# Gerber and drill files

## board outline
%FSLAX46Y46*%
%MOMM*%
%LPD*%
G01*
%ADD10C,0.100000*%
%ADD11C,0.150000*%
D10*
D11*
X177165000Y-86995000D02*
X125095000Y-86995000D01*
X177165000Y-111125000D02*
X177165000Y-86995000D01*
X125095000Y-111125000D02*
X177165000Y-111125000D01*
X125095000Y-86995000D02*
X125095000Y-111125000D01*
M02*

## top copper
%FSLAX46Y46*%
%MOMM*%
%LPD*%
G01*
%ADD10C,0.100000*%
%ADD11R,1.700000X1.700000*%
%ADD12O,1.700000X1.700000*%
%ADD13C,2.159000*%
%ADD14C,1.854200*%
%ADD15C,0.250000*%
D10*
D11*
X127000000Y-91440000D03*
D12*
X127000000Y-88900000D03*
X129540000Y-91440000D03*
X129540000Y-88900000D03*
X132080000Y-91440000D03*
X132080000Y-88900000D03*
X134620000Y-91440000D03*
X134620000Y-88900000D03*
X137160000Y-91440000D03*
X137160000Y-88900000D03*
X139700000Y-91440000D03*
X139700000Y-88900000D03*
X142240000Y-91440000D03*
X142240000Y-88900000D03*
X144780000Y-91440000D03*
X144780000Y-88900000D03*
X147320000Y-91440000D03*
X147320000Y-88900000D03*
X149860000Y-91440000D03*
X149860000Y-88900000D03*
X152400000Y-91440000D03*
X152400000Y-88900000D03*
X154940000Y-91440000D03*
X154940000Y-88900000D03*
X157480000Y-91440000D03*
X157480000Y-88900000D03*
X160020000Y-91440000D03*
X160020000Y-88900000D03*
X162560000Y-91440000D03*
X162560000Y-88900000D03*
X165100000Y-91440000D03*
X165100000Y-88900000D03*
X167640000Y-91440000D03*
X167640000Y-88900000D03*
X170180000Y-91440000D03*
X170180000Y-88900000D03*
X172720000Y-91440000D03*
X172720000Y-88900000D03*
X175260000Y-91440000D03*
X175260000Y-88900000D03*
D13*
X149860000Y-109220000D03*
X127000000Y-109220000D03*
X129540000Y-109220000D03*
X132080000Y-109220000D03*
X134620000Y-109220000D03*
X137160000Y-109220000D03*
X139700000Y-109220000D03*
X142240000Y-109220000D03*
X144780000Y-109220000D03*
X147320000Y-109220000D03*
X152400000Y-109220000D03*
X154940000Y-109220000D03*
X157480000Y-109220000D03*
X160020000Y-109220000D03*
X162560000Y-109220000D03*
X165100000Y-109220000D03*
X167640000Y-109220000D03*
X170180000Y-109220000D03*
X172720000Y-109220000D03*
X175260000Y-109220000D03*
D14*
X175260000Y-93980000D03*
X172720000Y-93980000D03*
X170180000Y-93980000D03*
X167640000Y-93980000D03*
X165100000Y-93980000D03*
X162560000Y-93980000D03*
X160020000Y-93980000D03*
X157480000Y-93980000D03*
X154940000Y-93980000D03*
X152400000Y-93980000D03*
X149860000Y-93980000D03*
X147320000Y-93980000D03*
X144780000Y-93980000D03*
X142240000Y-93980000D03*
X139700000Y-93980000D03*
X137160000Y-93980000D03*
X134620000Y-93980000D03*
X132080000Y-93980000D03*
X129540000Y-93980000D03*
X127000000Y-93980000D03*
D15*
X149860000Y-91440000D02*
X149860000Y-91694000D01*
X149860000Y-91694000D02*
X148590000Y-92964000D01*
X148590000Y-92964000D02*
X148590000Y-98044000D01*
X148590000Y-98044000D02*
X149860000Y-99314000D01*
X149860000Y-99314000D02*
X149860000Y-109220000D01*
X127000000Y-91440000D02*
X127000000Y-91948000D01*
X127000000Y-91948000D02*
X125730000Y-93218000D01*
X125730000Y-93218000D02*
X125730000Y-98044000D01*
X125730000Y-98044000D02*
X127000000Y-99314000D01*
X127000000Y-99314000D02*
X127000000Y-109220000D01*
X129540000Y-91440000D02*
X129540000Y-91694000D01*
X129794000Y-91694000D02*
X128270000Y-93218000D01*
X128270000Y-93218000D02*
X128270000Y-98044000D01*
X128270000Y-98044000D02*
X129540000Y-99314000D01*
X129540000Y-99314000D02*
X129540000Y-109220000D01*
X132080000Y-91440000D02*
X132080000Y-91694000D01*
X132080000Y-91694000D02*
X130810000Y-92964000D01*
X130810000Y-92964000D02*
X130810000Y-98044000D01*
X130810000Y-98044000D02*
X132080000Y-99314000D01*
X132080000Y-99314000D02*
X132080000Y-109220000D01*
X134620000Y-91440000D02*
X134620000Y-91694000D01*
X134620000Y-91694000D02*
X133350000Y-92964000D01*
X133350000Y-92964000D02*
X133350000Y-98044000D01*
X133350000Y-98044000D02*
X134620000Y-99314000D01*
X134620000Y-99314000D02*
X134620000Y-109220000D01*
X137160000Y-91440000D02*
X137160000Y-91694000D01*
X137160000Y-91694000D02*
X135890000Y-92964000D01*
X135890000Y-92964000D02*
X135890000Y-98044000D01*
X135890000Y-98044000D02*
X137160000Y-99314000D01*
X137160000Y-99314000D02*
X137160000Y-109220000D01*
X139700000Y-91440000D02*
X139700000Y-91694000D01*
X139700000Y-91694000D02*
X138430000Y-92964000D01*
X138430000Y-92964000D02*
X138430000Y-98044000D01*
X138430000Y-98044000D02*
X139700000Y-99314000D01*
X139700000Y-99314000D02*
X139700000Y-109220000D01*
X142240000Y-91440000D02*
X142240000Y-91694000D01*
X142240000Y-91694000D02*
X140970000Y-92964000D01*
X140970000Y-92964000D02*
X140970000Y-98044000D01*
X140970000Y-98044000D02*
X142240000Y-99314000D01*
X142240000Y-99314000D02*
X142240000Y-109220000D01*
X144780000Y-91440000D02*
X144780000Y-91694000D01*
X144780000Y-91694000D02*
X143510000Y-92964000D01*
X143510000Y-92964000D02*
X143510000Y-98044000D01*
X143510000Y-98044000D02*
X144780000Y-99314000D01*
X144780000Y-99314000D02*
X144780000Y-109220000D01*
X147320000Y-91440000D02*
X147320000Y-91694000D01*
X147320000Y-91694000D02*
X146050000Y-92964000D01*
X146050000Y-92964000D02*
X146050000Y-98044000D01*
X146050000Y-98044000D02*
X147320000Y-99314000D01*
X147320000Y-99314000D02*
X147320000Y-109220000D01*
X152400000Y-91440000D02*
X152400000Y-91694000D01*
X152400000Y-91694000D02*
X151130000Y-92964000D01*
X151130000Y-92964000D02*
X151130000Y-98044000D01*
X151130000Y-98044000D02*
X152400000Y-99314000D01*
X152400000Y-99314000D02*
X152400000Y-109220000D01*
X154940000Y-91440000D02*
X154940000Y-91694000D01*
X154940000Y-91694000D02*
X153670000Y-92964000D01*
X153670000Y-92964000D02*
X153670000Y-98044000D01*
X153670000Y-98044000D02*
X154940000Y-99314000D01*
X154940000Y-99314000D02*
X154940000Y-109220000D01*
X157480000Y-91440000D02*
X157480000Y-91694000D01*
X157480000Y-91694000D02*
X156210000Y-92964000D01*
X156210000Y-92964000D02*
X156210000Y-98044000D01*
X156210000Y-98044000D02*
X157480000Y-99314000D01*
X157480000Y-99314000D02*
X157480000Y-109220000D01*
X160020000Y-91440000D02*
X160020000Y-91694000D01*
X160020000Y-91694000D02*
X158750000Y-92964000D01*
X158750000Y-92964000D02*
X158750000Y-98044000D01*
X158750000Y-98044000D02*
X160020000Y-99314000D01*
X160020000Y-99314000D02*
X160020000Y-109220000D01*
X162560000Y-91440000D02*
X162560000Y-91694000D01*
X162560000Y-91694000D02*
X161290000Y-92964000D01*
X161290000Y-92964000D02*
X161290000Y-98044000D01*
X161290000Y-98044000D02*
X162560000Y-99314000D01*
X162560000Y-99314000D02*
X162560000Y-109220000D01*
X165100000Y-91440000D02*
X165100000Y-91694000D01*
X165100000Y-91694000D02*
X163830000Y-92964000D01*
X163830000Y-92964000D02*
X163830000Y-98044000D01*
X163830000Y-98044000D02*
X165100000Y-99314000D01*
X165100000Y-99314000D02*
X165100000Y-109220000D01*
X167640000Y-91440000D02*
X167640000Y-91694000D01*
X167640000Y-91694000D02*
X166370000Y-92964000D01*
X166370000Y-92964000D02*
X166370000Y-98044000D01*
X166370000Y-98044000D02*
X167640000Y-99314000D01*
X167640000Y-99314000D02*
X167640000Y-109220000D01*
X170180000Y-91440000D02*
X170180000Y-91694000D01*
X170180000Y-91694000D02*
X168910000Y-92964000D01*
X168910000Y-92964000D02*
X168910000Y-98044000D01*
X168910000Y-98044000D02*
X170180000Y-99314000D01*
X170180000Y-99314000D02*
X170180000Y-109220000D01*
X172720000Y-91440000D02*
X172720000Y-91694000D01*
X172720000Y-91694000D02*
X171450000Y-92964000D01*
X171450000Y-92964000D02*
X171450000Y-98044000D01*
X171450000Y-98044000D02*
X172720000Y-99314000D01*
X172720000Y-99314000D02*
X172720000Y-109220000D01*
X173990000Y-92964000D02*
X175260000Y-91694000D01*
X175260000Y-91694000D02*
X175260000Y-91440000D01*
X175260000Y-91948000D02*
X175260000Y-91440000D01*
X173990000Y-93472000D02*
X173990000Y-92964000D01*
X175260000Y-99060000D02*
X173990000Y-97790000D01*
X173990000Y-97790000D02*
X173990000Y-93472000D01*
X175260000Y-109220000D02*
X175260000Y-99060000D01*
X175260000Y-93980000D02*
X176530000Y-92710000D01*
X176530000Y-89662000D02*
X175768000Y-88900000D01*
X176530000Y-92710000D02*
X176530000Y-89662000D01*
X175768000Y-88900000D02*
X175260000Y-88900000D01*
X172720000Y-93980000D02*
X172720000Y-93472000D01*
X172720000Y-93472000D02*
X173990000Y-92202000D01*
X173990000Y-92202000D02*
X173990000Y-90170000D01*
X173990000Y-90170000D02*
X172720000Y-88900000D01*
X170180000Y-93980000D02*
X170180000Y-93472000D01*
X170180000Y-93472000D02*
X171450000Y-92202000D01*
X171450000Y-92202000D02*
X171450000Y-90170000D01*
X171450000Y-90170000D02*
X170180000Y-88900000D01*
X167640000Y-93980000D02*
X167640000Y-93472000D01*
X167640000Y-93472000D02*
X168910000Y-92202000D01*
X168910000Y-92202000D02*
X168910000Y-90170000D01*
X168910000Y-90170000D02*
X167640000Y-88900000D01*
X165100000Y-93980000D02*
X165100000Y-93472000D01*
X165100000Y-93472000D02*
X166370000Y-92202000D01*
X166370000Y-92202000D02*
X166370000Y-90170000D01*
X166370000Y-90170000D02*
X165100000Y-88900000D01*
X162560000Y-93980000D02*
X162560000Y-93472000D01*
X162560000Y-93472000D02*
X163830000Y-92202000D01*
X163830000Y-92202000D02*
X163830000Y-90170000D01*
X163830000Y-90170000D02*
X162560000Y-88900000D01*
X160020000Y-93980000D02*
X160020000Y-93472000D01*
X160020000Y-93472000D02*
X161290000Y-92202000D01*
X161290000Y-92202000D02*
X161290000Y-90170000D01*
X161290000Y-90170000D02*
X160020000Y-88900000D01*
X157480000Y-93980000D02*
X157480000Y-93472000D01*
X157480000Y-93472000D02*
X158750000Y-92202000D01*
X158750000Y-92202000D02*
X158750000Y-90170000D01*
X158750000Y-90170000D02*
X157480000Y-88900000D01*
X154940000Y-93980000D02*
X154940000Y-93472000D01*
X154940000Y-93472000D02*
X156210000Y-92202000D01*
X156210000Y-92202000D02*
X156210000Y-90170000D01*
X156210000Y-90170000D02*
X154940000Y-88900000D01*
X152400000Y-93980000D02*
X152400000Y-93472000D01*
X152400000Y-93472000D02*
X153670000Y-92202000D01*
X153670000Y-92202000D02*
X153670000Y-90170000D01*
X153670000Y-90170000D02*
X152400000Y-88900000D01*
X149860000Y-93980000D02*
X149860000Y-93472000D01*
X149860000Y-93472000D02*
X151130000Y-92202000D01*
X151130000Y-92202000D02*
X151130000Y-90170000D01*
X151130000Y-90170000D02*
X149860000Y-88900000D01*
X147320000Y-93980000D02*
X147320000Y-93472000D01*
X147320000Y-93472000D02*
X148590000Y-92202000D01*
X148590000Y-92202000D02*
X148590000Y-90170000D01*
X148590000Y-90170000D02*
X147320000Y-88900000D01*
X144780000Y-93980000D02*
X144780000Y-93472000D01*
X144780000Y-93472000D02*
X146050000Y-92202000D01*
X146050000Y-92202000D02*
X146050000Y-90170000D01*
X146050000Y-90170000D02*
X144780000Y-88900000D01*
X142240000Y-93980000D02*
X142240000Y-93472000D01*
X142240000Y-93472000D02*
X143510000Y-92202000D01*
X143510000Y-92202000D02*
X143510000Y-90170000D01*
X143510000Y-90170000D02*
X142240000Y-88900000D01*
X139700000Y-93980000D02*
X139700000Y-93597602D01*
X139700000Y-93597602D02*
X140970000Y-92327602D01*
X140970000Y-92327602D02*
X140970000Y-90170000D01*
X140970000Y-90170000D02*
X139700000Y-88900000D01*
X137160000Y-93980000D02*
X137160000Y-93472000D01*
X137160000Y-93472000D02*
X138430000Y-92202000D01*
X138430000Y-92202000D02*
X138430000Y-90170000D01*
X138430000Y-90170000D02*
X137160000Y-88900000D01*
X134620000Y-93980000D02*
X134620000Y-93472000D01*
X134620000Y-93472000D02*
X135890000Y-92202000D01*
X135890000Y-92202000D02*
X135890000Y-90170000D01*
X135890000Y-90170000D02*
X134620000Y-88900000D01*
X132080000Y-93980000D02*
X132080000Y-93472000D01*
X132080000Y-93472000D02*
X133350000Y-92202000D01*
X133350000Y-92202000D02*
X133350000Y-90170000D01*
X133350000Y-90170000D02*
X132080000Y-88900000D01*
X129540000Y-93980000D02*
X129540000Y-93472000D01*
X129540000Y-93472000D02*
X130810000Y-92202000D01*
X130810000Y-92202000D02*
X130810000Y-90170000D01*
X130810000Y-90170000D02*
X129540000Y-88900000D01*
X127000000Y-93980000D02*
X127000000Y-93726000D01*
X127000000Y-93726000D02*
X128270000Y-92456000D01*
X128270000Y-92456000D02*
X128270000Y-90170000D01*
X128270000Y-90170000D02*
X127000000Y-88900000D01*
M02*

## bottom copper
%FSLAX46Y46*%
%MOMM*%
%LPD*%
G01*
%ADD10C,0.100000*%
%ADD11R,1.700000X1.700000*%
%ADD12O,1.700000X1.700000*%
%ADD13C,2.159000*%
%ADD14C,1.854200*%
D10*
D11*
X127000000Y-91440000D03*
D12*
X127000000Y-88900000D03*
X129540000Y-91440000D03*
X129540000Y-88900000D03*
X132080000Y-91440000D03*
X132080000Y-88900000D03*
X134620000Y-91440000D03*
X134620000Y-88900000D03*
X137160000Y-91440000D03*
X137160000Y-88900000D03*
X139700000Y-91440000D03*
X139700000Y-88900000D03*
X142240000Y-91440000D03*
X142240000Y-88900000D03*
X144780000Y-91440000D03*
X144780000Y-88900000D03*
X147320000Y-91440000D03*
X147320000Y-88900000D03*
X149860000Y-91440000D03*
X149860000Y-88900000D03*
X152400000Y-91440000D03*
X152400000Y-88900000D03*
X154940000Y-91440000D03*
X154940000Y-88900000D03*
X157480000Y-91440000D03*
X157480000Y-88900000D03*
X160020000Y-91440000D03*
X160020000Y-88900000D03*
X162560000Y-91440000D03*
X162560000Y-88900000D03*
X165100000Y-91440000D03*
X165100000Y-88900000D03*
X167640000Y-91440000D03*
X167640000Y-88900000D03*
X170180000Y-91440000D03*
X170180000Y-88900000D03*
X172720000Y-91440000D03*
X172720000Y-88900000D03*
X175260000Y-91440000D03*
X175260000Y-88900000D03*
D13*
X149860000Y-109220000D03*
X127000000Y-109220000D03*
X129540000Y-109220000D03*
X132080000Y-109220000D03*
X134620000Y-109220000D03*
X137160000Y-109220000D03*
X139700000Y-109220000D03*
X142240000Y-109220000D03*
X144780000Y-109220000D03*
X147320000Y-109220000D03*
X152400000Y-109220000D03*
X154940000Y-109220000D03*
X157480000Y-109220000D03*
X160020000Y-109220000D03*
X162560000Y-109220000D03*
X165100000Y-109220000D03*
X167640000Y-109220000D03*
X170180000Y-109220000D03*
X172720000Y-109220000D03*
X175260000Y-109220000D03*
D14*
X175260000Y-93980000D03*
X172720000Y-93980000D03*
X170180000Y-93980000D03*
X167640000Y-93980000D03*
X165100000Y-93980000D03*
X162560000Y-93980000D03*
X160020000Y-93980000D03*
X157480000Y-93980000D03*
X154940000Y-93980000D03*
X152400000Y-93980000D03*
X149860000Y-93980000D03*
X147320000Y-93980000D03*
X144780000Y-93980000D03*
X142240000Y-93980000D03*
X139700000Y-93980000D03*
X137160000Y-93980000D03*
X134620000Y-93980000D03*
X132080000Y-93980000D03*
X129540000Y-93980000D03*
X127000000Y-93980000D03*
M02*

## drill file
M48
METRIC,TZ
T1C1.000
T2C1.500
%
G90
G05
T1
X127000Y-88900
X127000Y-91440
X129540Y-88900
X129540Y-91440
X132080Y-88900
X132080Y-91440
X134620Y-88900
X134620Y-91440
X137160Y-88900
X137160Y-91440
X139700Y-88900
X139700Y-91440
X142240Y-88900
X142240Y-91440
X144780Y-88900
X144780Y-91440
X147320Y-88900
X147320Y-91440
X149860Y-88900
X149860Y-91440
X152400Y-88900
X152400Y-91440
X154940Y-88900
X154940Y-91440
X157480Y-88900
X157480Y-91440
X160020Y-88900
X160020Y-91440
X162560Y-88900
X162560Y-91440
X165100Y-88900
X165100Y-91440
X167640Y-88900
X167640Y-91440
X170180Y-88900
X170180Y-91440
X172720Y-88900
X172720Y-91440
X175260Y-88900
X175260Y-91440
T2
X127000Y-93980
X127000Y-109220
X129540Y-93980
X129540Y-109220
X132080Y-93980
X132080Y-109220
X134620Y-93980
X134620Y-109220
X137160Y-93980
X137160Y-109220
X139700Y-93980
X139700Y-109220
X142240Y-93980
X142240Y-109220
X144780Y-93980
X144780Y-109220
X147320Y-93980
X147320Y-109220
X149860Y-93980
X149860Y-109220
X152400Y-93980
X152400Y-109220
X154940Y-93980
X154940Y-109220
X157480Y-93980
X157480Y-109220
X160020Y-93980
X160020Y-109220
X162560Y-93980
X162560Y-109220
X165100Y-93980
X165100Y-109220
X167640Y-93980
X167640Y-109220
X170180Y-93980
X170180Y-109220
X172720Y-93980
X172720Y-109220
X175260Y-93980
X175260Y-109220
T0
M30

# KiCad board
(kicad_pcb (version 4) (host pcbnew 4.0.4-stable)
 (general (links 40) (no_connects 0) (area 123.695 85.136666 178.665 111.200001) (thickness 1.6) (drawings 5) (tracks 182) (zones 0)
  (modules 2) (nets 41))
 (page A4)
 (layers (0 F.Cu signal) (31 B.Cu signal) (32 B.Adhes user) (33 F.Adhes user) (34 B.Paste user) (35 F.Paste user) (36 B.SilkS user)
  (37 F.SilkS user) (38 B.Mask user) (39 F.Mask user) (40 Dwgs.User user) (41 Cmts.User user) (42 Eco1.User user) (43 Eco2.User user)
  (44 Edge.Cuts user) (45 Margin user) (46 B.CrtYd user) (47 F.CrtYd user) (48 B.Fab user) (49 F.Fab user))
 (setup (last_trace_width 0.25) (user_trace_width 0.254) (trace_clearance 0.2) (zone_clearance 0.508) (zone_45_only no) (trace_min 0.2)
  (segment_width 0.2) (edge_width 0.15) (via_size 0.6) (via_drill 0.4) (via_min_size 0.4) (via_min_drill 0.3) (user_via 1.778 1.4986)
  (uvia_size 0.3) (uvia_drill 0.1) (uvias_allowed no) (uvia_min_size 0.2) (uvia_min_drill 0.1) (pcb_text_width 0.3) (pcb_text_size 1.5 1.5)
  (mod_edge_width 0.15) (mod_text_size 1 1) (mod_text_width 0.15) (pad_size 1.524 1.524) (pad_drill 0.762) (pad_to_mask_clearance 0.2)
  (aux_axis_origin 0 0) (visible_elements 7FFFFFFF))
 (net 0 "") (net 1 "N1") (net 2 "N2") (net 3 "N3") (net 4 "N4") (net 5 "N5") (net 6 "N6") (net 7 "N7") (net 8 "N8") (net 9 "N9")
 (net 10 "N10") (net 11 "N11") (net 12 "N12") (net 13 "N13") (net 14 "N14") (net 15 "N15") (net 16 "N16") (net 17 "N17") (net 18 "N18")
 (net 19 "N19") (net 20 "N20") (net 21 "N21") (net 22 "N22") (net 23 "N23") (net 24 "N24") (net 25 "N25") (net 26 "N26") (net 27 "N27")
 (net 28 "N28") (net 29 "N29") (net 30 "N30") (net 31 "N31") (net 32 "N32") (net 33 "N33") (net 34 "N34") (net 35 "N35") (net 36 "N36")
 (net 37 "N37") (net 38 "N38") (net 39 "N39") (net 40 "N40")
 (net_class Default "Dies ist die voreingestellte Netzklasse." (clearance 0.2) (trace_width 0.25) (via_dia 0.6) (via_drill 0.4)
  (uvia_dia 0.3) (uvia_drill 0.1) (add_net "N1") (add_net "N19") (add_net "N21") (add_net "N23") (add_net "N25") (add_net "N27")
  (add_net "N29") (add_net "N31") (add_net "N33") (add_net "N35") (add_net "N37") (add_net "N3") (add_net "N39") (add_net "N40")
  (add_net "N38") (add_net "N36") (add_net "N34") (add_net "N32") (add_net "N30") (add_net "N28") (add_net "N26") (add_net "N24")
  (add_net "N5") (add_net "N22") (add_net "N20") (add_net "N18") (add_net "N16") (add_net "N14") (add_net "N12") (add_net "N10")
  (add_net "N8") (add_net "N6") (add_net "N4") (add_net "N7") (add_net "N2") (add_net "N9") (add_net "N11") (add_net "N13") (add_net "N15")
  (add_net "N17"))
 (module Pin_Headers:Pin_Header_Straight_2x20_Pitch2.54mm (layer F.Cu) (at 127 91.44 90)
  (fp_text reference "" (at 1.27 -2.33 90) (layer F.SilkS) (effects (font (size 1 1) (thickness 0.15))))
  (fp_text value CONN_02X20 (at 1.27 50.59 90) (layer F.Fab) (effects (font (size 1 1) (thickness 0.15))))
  (pad 1 thru_hole rect (at 0 0 90) (size 1.7 1.7) (drill 1) (layers *.Cu *.Mask) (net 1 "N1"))
  (pad 2 thru_hole oval (at 2.54 0 90) (size 1.7 1.7) (drill 1) (layers *.Cu *.Mask) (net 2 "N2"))
  (pad 3 thru_hole oval (at 0 2.54 90) (size 1.7 1.7) (drill 1) (layers *.Cu *.Mask) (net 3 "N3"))
  (pad 4 thru_hole oval (at 2.54 2.54 90) (size 1.7 1.7) (drill 1) (layers *.Cu *.Mask) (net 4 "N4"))
  (pad 5 thru_hole oval (at 0 5.08 90) (size 1.7 1.7) (drill 1) (layers *.Cu *.Mask) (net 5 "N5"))
  (pad 6 thru_hole oval (at 2.54 5.08 90) (size 1.7 1.7) (drill 1) (layers *.Cu *.Mask) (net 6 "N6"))
  (pad 7 thru_hole oval (at 0 7.62 90) (size 1.7 1.7) (drill 1) (layers *.Cu *.Mask) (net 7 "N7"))
  (pad 8 thru_hole oval (at 2.54 7.62 90) (size 1.7 1.7) (drill 1) (layers *.Cu *.Mask) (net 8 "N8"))
  (pad 9 thru_hole oval (at 0 10.16 90) (size 1.7 1.7) (drill 1) (layers *.Cu *.Mask) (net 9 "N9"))
  (pad 10 thru_hole oval (at 2.54 10.16 90) (size 1.7 1.7) (drill 1) (layers *.Cu *.Mask) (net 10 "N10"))
  (pad 11 thru_hole oval (at 0 12.7 90) (size 1.7 1.7) (drill 1) (layers *.Cu *.Mask) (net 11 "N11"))
  (pad 12 thru_hole oval (at 2.54 12.7 90) (size 1.7 1.7) (drill 1) (layers *.Cu *.Mask) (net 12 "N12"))
  (pad 13 thru_hole oval (at 0 15.24 90) (size 1.7 1.7) (drill 1) (layers *.Cu *.Mask) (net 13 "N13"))
  (pad 14 thru_hole oval (at 2.54 15.24 90) (size 1.7 1.7) (drill 1) (layers *.Cu *.Mask) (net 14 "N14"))
  (pad 15 thru_hole oval (at 0 17.78 90) (size 1.7 1.7) (drill 1) (layers *.Cu *.Mask) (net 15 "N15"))
  (pad 16 thru_hole oval (at 2.54 17.78 90) (size 1.7 1.7) (drill 1) (layers *.Cu *.Mask) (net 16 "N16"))
  (pad 17 thru_hole oval (at 0 20.32 90) (size 1.7 1.7) (drill 1) (layers *.Cu *.Mask) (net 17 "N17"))
  (pad 18 thru_hole oval (at 2.54 20.32 90) (size 1.7 1.7) (drill 1) (layers *.Cu *.Mask) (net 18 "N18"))
  (pad 19 thru_hole oval (at 0 22.86 90) (size 1.7 1.7) (drill 1) (layers *.Cu *.Mask) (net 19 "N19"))
  (pad 20 thru_hole oval (at 2.54 22.86 90) (size 1.7 1.7) (drill 1) (layers *.Cu *.Mask) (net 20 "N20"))
  (pad 21 thru_hole oval (at 0 25.4 90) (size 1.7 1.7) (drill 1) (layers *.Cu *.Mask) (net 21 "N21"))
  (pad 22 thru_hole oval (at 2.54 25.4 90) (size 1.7 1.7) (drill 1) (layers *.Cu *.Mask) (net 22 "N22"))
  (pad 23 thru_hole oval (at 0 27.94 90) (size 1.7 1.7) (drill 1) (layers *.Cu *.Mask) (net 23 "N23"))
  (pad 24 thru_hole oval (at 2.54 27.94 90) (size 1.7 1.7) (drill 1) (layers *.Cu *.Mask) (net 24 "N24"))
  (pad 25 thru_hole oval (at 0 30.48 90) (size 1.7 1.7) (drill 1) (layers *.Cu *.Mask) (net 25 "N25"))
  (pad 26 thru_hole oval (at 2.54 30.48 90) (size 1.7 1.7) (drill 1) (layers *.Cu *.Mask) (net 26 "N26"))
  (pad 27 thru_hole oval (at 0 33.02 90) (size 1.7 1.7) (drill 1) (layers *.Cu *.Mask) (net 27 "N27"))
  (pad 28 thru_hole oval (at 2.54 33.02 90) (size 1.7 1.7) (drill 1) (layers *.Cu *.Mask) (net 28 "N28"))
  (pad 29 thru_hole oval (at 0 35.56 90) (size 1.7 1.7) (drill 1) (layers *.Cu *.Mask) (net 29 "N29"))
  (pad 30 thru_hole oval (at 2.54 35.56 90) (size 1.7 1.7) (drill 1) (layers *.Cu *.Mask) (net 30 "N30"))
  (pad 31 thru_hole oval (at 0 38.1 90) (size 1.7 1.7) (drill 1) (layers *.Cu *.Mask) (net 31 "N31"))
  (pad 32 thru_hole oval (at 2.54 38.1 90) (size 1.7 1.7) (drill 1) (layers *.Cu *.Mask) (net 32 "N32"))
  (pad 33 thru_hole oval (at 0 40.64 90) (size 1.7 1.7) (drill 1) (layers *.Cu *.Mask) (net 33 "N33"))
  (pad 34 thru_hole oval (at 2.54 40.64 90) (size 1.7 1.7) (drill 1) (layers *.Cu *.Mask) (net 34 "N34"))
  (pad 35 thru_hole oval (at 0 43.18 90) (size 1.7 1.7) (drill 1) (layers *.Cu *.Mask) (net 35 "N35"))
  (pad 36 thru_hole oval (at 2.54 43.18 90) (size 1.7 1.7) (drill 1) (layers *.Cu *.Mask) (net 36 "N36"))
  (pad 37 thru_hole oval (at 0 45.72 90) (size 1.7 1.7) (drill 1) (layers *.Cu *.Mask) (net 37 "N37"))
  (pad 38 thru_hole oval (at 2.54 45.72 90) (size 1.7 1.7) (drill 1) (layers *.Cu *.Mask) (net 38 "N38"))
  (pad 39 thru_hole oval (at 0 48.26 90) (size 1.7 1.7) (drill 1) (layers *.Cu *.Mask) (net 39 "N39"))
  (pad 40 thru_hole oval (at 2.54 48.26 90) (size 1.7 1.7) (drill 1) (layers *.Cu *.Mask) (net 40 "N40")))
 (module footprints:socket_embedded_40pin (layer F.Cu) (at 149.86 101.6)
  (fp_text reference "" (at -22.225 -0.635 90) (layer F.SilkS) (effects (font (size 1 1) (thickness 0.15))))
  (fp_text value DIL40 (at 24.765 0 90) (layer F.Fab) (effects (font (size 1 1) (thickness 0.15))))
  (pad 10 thru_hole circle (at 0 7.62) (size 2.159 2.159) (drill 1.5) (layers *.Cu *.Mask) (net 19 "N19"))
  (pad 1 thru_hole circle (at -22.86 7.62) (size 2.159 2.159) (drill 1.5) (layers *.Cu *.Mask) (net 1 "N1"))
  (pad 2 thru_hole circle (at -20.32 7.62) (size 2.159 2.159) (drill 1.5) (layers *.Cu *.Mask) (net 3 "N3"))
  (pad 3 thru_hole circle (at -17.78 7.62) (size 2.159 2.159) (drill 1.5) (layers *.Cu *.Mask) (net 5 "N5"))
  (pad 4 thru_hole circle (at -15.24 7.62) (size 2.159 2.159) (drill 1.5) (layers *.Cu *.Mask) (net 7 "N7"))
  (pad 5 thru_hole circle (at -12.7 7.62) (size 2.159 2.159) (drill 1.5) (layers *.Cu *.Mask) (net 9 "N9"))
  (pad 6 thru_hole circle (at -10.16 7.62) (size 2.159 2.159) (drill 1.5) (layers *.Cu *.Mask) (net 11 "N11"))
  (pad 7 thru_hole circle (at -7.62 7.62) (size 2.159 2.159) (drill 1.5) (layers *.Cu *.Mask) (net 13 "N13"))
  (pad 8 thru_hole circle (at -5.08 7.62) (size 2.159 2.159) (drill 1.5) (layers *.Cu *.Mask) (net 15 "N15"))
  (pad 9 thru_hole circle (at -2.54 7.62) (size 2.159 2.159) (drill 1.5) (layers *.Cu *.Mask) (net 17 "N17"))
  (pad 11 thru_hole circle (at 2.54 7.62) (size 2.159 2.159) (drill 1.5) (layers *.Cu *.Mask) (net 21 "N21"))
  (pad 12 thru_hole circle (at 5.08 7.62) (size 2.159 2.159) (drill 1.5) (layers *.Cu *.Mask) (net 23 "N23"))
  (pad 13 thru_hole circle (at 7.62 7.62) (size 2.159 2.159) (drill 1.5) (layers *.Cu *.Mask) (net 25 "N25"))
  (pad 14 thru_hole circle (at 10.16 7.62) (size 2.159 2.159) (drill 1.5) (layers *.Cu *.Mask) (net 27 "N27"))
  (pad 15 thru_hole circle (at 12.7 7.62) (size 2.159 2.159) (drill 1.5) (layers *.Cu *.Mask) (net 29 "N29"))
  (pad 16 thru_hole circle (at 15.24 7.62) (size 2.159 2.159) (drill 1.5) (layers *.Cu *.Mask) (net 31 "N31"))
  (pad 17 thru_hole circle (at 17.78 7.62) (size 2.159 2.159) (drill 1.5) (layers *.Cu *.Mask) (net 33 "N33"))
  (pad 18 thru_hole circle (at 20.32 7.62) (size 2.159 2.159) (drill 1.5) (layers *.Cu *.Mask) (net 35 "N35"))
  (pad 19 thru_hole circle (at 22.86 7.62) (size 2.159 2.159) (drill 1.5) (layers *.Cu *.Mask) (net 37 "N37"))
  (pad 20 thru_hole circle (at 25.4 7.62) (size 2.159 2.159) (drill 1.5) (layers *.Cu *.Mask) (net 39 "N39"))
  (pad 21 thru_hole circle (at 25.4 -7.62) (size 1.8542 1.8542) (drill 1.5) (layers *.Cu *.Mask) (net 40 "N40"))
  (pad 22 thru_hole circle (at 22.86 -7.62) (size 1.8542 1.8542) (drill 1.5) (layers *.Cu *.Mask) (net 38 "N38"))
  (pad 23 thru_hole circle (at 20.32 -7.62) (size 1.8542 1.8542) (drill 1.5) (layers *.Cu *.Mask) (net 36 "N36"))
  (pad 24 thru_hole circle (at 17.78 -7.62) (size 1.8542 1.8542) (drill 1.5) (layers *.Cu *.Mask) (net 34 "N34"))
  (pad 25 thru_hole circle (at 15.24 -7.62) (size 1.8542 1.8542) (drill 1.5) (layers *.Cu *.Mask) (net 32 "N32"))
  (pad 26 thru_hole circle (at 12.7 -7.62) (size 1.8542 1.8542) (drill 1.5) (layers *.Cu *.Mask) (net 30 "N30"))
  (pad 27 thru_hole circle (at 10.16 -7.62) (size 1.8542 1.8542) (drill 1.5) (layers *.Cu *.Mask) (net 28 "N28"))
  (pad 28 thru_hole circle (at 7.62 -7.62) (size 1.8542 1.8542) (drill 1.5) (layers *.Cu *.Mask) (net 26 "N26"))
  (pad 29 thru_hole circle (at 5.08 -7.62) (size 1.8542 1.8542) (drill 1.5) (layers *.Cu *.Mask) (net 24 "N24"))
  (pad 30 thru_hole circle (at 2.54 -7.62) (size 1.8542 1.8542) (drill 1.5) (layers *.Cu *.Mask) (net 22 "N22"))
  (pad 31 thru_hole circle (at 0 -7.62) (size 1.8542 1.8542) (drill 1.5) (layers *.Cu *.Mask) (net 20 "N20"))
  (pad 32 thru_hole circle (at -2.54 -7.62) (size 1.8542 1.8542) (drill 1.5) (layers *.Cu *.Mask) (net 18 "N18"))
  (pad 33 thru_hole circle (at -5.08 -7.62) (size 1.8542 1.8542) (drill 1.5) (layers *.Cu *.Mask) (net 16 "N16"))
  (pad 34 thru_hole circle (at -7.62 -7.62) (size 1.8542 1.8542) (drill 1.5) (layers *.Cu *.Mask) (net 14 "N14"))
  (pad 35 thru_hole circle (at -10.16 -7.62) (size 1.8542 1.8542) (drill 1.5) (layers *.Cu *.Mask) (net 12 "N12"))
  (pad 36 thru_hole circle (at -12.7 -7.62) (size 1.8542 1.8542) (drill 1.5) (layers *.Cu *.Mask) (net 10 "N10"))
  (pad 37 thru_hole circle (at -15.24 -7.62) (size 1.8542 1.8542) (drill 1.5) (layers *.Cu *.Mask) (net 8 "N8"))
  (pad 38 thru_hole circle (at -17.78 -7.62) (size 1.8542 1.8542) (drill 1.5) (layers *.Cu *.Mask) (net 6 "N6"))
  (pad 39 thru_hole circle (at -20.32 -7.62) (size 1.8542 1.8542) (drill 1.5) (layers *.Cu *.Mask) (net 4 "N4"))
  (pad 40 thru_hole circle (at -22.86 -7.62) (size 1.8542 1.8542) (drill 1.5) (layers *.Cu *.Mask) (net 2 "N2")))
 (gr_line (start 177.165 86.995) (end 125.095 86.995) (angle 90) (layer Edge.Cuts) (width 0.15))
 (gr_line (start 177.165 111.125) (end 177.165 86.995) (angle 90) (layer Edge.Cuts) (width 0.15))
 (gr_line (start 125.095 111.125) (end 177.165 111.125) (angle 90) (layer Edge.Cuts) (width 0.15))
 (gr_line (start 125.095 86.995) (end 125.095 111.125) (angle 90) (layer Edge.Cuts) (width 0.15))
 (segment (start 149.86 91.44) (end 149.86 91.694) (width 0.25) (layer F.Cu) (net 19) (status C00000))
 (segment (start 149.86 91.694) (end 148.59 92.964) (width 0.25) (layer F.Cu) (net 19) (status 400000))
 (segment (start 148.59 92.964) (end 148.59 98.044) (width 0.25) (layer F.Cu) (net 19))
 (segment (start 148.59 98.044) (end 149.86 99.314) (width 0.25) (layer F.Cu) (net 19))
 (segment (start 149.86 99.314) (end 149.86 109.22) (width 0.25) (layer F.Cu) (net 19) (status 800000))
 (segment (start 127 91.44) (end 127 91.948) (width 0.25) (layer F.Cu) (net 1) (status C00000))
 (segment (start 127 91.948) (end 125.73 93.218) (width 0.25) (layer F.Cu) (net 1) (status 400000))
 (segment (start 125.73 93.218) (end 125.73 98.044) (width 0.25) (layer F.Cu) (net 1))
 (segment (start 125.73 98.044) (end 127 99.314) (width 0.25) (layer F.Cu) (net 1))
 (segment (start 127 99.314) (end 127 109.22) (width 0.25) (layer F.Cu) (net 1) (status 800000))
 (segment (start 129.54 91.44) (end 129.54 91.694) (width 0.25) (layer F.Cu) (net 3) (status C00000))
 (segment (start 129.794 91.694) (end 128.27 93.218) (width 0.25) (layer F.Cu) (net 3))
 (segment (start 128.27 93.218) (end 128.27 98.044) (width 0.25) (layer F.Cu) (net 3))
 (segment (start 128.27 98.044) (end 129.54 99.314) (width 0.25) (layer F.Cu) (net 3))
 (segment (start 129.54 99.314) (end 129.54 109.22) (width 0.25) (layer F.Cu) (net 3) (status 800000))
 (segment (start 132.08 91.44) (end 132.08 91.694) (width 0.25) (layer F.Cu) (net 5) (status C00000))
 (segment (start 132.08 91.694) (end 130.81 92.964) (width 0.25) (layer F.Cu) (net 5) (status 400000))
 (segment (start 130.81 92.964) (end 130.81 98.044) (width 0.25) (layer F.Cu) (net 5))
 (segment (start 130.81 98.044) (end 132.08 99.314) (width 0.25) (layer F.Cu) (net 5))
 (segment (start 132.08 99.314) (end 132.08 109.22) (width 0.25) (layer F.Cu) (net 5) (status 800000))
 (segment (start 134.62 91.44) (end 134.62 91.694) (width 0.25) (layer F.Cu) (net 7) (status C00000))
 (segment (start 134.62 91.694) (end 133.35 92.964) (width 0.25) (layer F.Cu) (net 7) (status 400000))
 (segment (start 133.35 92.964) (end 133.35 98.044) (width 0.25) (layer F.Cu) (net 7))
 (segment (start 133.35 98.044) (end 134.62 99.314) (width 0.25) (layer F.Cu) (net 7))
 (segment (start 134.62 99.314) (end 134.62 109.22) (width 0.25) (layer F.Cu) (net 7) (status 800000))
 (segment (start 137.16 91.44) (end 137.16 91.694) (width 0.25) (layer F.Cu) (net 9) (status C00000))
 (segment (start 137.16 91.694) (end 135.89 92.964) (width 0.25) (layer F.Cu) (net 9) (status 400000))
 (segment (start 135.89 92.964) (end 135.89 98.044) (width 0.25) (layer F.Cu) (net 9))
 (segment (start 135.89 98.044) (end 137.16 99.314) (width 0.25) (layer F.Cu) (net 9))
 (segment (start 137.16 99.314) (end 137.16 109.22) (width 0.25) (layer F.Cu) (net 9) (status 800000))
 (segment (start 139.7 91.44) (end 139.7 91.694) (width 0.25) (layer F.Cu) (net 11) (status C00000))
 (segment (start 139.7 91.694) (end 138.43 92.964) (width 0.25) (layer F.Cu) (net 11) (status 400000))
 (segment (start 138.43 92.964) (end 138.43 98.044) (width 0.25) (layer F.Cu) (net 11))
 (segment (start 138.43 98.044) (end 139.7 99.314) (width 0.25) (layer F.Cu) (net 11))
 (segment (start 139.7 99.314) (end 139.7 109.22) (width 0.25) (layer F.Cu) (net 11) (status 800000))
 (segment (start 142.24 91.44) (end 142.24 91.694) (width 0.25) (layer F.Cu) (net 13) (status C00000))
 (segment (start 142.24 91.694) (end 140.97 92.964) (width 0.25) (layer F.Cu) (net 13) (status 400000))
 (segment (start 140.97 92.964) (end 140.97 98.044) (width 0.25) (layer F.Cu) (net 13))
 (segment (start 140.97 98.044) (end 142.24 99.314) (width 0.25) (layer F.Cu) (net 13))
 (segment (start 142.24 99.314) (end 142.24 109.22) (width 0.25) (layer F.Cu) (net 13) (status 800000))
 (segment (start 144.78 91.44) (end 144.78 91.694) (width 0.25) (layer F.Cu) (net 15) (status C00000))
 (segment (start 144.78 91.694) (end 143.51 92.964) (width 0.25) (layer F.Cu) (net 15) (status 400000))
 (segment (start 143.51 92.964) (end 143.51 98.044) (width 0.25) (layer F.Cu) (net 15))
 (segment (start 143.51 98.044) (end 144.78 99.314) (width 0.25) (layer F.Cu) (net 15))
 (segment (start 144.78 99.314) (end 144.78 109.22) (width 0.25) (layer F.Cu) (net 15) (status 800000))
 (segment (start 147.32 91.44) (end 147.32 91.694) (width 0.25) (layer F.Cu) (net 17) (status C00000))
 (segment (start 147.32 91.694) (end 146.05 92.964) (width 0.25) (layer F.Cu) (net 17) (status 400000))
 (segment (start 146.05 92.964) (end 146.05 98.044) (width 0.25) (layer F.Cu) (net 17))
 (segment (start 146.05 98.044) (end 147.32 99.314) (width 0.25) (layer F.Cu) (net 17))
 (segment (start 147.32 99.314) (end 147.32 109.22) (width 0.25) (layer F.Cu) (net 17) (status 800000))
 (segment (start 152.4 91.44) (end 152.4 91.694) (width 0.25) (layer F.Cu) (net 21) (status C00000))
 (segment (start 152.4 91.694) (end 151.13 92.964) (width 0.25) (layer F.Cu) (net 21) (status 400000))
 (segment (start 151.13 92.964) (end 151.13 98.044) (width 0.25) (layer F.Cu) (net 21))
 (segment (start 151.13 98.044) (end 152.4 99.314) (width 0.25) (layer F.Cu) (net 21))
 (segment (start 152.4 99.314) (end 152.4 109.22) (width 0.25) (layer F.Cu) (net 21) (status 800000))
 (segment (start 154.94 91.44) (end 154.94 91.694) (width 0.25) (layer F.Cu) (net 23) (status C00000))
 (segment (start 154.94 91.694) (end 153.67 92.964) (width 0.25) (layer F.Cu) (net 23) (status 400000))
 (segment (start 153.67 92.964) (end 153.67 98.044) (width 0.25) (layer F.Cu) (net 23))
 (segment (start 153.67 98.044) (end 154.94 99.314) (width 0.25) (layer F.Cu) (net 23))
 (segment (start 154.94 99.314) (end 154.94 109.22) (width 0.25) (layer F.Cu) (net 23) (status 800000))
 (segment (start 157.48 91.44) (end 157.48 91.694) (width 0.25) (layer F.Cu) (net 25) (status C00000))
 (segment (start 157.48 91.694) (end 156.21 92.964) (width 0.25) (layer F.Cu) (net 25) (status 400000))
 (segment (start 156.21 92.964) (end 156.21 98.044) (width 0.25) (layer F.Cu) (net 25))
 (segment (start 156.21 98.044) (end 157.48 99.314) (width 0.25) (layer F.Cu) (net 25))
 (segment (start 157.48 99.314) (end 157.48 109.22) (width 0.25) (layer F.Cu) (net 25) (status 800000))
 (segment (start 160.02 91.44) (end 160.02 91.694) (width 0.25) (layer F.Cu) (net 27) (status C00000))
 (segment (start 160.02 91.694) (end 158.75 92.964) (width 0.25) (layer F.Cu) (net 27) (status 400000))
 (segment (start 158.75 92.964) (end 158.75 98.044) (width 0.25) (layer F.Cu) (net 27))
 (segment (start 158.75 98.044) (end 160.02 99.314) (width 0.25) (layer F.Cu) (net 27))
 (segment (start 160.02 99.314) (end 160.02 109.22) (width 0.25) (layer F.Cu) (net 27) (status 800000))
 (segment (start 162.56 91.44) (end 162.56 91.694) (width 0.25) (layer F.Cu) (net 29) (status C00000))
 (segment (start 162.56 91.694) (end 161.29 92.964) (width 0.25) (layer F.Cu) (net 29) (status 400000))
 (segment (start 161.29 92.964) (end 161.29 98.044) (width 0.25) (layer F.Cu) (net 29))
 (segment (start 161.29 98.044) (end 162.56 99.314) (width 0.25) (layer F.Cu) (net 29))
 (segment (start 162.56 99.314) (end 162.56 109.22) (width 0.25) (layer F.Cu) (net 29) (status 800000))
 (segment (start 165.1 91.44) (end 165.1 91.694) (width 0.25) (layer F.Cu) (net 31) (status C00000))
 (segment (start 165.1 91.694) (end 163.83 92.964) (width 0.25) (layer F.Cu) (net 31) (status 400000))
 (segment (start 163.83 92.964) (end 163.83 98.044) (width 0.25) (layer F.Cu) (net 31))
 (segment (start 163.83 98.044) (end 165.1 99.314) (width 0.25) (layer F.Cu) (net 31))
 (segment (start 165.1 99.314) (end 165.1 109.22) (width 0.25) (layer F.Cu) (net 31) (status 800000))
 (segment (start 167.64 91.44) (end 167.64 91.694) (width 0.25) (layer F.Cu) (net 33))
 (segment (start 167.64 91.694) (end 166.37 92.964) (width 0.25) (layer F.Cu) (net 33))
 (segment (start 166.37 92.964) (end 166.37 98.044) (width 0.25) (layer F.Cu) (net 33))
 (segment (start 166.37 98.044) (end 167.64 99.314) (width 0.25) (layer F.Cu) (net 33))
 (segment (start 167.64 99.314) (end 167.64 109.22) (width 0.25) (layer F.Cu) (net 33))
 (segment (start 170.18 91.44) (end 170.18 91.694) (width 0.25) (layer F.Cu) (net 35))
 (segment (start 170.18 91.694) (end 168.91 92.964) (width 0.25) (layer F.Cu) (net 35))
 (segment (start 168.91 92.964) (end 168.91 98.044) (width 0.25) (layer F.Cu) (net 35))
 (segment (start 168.91 98.044) (end 170.18 99.314) (width 0.25) (layer F.Cu) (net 35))
 (segment (start 170.18 99.314) (end 170.18 109.22) (width 0.25) (layer F.Cu) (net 35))
 (segment (start 172.72 91.44) (end 172.72 91.694) (width 0.25) (layer F.Cu) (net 37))
 (segment (start 172.72 91.694) (end 171.45 92.964) (width 0.25) (layer F.Cu) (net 37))
 (segment (start 171.45 92.964) (end 171.45 98.044) (width 0.25) (layer F.Cu) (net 37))
 (segment (start 171.45 98.044) (end 172.72 99.314) (width 0.25) (layer F.Cu) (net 37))
 (segment (start 172.72 99.314) (end 172.72 109.22) (width 0.25) (layer F.Cu) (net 37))
 (segment (start 173.99 92.964) (end 175.26 91.694) (width 0.25) (layer F.Cu) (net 39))
 (segment (start 175.26 91.694) (end 175.26 91.44) (width 0.25) (layer F.Cu) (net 39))
 (segment (start 175.26 91.948) (end 175.26 91.44) (width 0.25) (layer F.Cu) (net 39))
 (segment (start 173.99 93.472) (end 173.99 92.964) (width 0.25) (layer F.Cu) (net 39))
 (segment (start 175.26 99.06) (end 173.99 97.79) (width 0.25) (layer F.Cu) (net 39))
 (segment (start 173.99 97.79) (end 173.99 93.472) (width 0.25) (layer F.Cu) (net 39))
 (segment (start 175.26 109.22) (end 175.26 99.06) (width 0.25) (layer F.Cu) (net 39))
 (segment (start 175.26 93.98) (end 176.53 92.71) (width 0.25) (layer F.Cu) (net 40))
 (segment (start 176.53 89.662) (end 175.768 88.9) (width 0.25) (layer F.Cu) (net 40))
 (segment (start 176.53 92.71) (end 176.53 89.662) (width 0.25) (layer F.Cu) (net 40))
 (segment (start 175.768 88.9) (end 175.26 88.9) (width 0.25) (layer F.Cu) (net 40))
 (segment (start 172.72 93.98) (end 172.72 93.472) (width 0.25) (layer F.Cu) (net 38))
 (segment (start 172.72 93.472) (end 173.99 92.202) (width 0.25) (layer F.Cu) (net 38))
 (segment (start 173.99 92.202) (end 173.99 90.17) (width 0.25) (layer F.Cu) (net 38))
 (segment (start 173.99 90.17) (end 172.72 88.9) (width 0.25) (layer F.Cu) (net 38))
 (segment (start 170.18 93.98) (end 170.18 93.472) (width 0.25) (layer F.Cu) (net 36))
 (segment (start 170.18 93.472) (end 171.45 92.202) (width 0.25) (layer F.Cu) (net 36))
 (segment (start 171.45 92.202) (end 171.45 90.17) (width 0.25) (layer F.Cu) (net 36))
 (segment (start 171.45 90.17) (end 170.18 88.9) (width 0.25) (layer F.Cu) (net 36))
 (segment (start 167.64 93.98) (end 167.64 93.472) (width 0.25) (layer F.Cu) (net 34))
 (segment (start 167.64 93.472) (end 168.91 92.202) (width 0.25) (layer F.Cu) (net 34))
 (segment (start 168.91 92.202) (end 168.91 90.17) (width 0.25) (layer F.Cu) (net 34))
 (segment (start 168.91 90.17) (end 167.64 88.9) (width 0.25) (layer F.Cu) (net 34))
 (segment (start 165.1 93.98) (end 165.1 93.472) (width 0.25) (layer F.Cu) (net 32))
 (segment (start 165.1 93.472) (end 166.37 92.202) (width 0.25) (layer F.Cu) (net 32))
 (segment (start 166.37 92.202) (end 166.37 90.17) (width 0.25) (layer F.Cu) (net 32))
 (segment (start 166.37 90.17) (end 165.1 88.9) (width 0.25) (layer F.Cu) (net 32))
 (segment (start 162.56 93.98) (end 162.56 93.472) (width 0.25) (layer F.Cu) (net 30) (status C00000))
 (segment (start 162.56 93.472) (end 163.83 92.202) (width 0.25) (layer F.Cu) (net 30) (status 400000))
 (segment (start 163.83 92.202) (end 163.83 90.17) (width 0.25) (layer F.Cu) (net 30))
 (segment (start 163.83 90.17) (end 162.56 88.9) (width 0.25) (layer F.Cu) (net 30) (status 800000))
 (segment (start 160.02 93.98) (end 160.02 93.472) (width 0.25) (layer F.Cu) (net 28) (status C00000))
 (segment (start 160.02 93.472) (end 161.29 92.202) (width 0.25) (layer F.Cu) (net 28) (status 400000))
 (segment (start 161.29 92.202) (end 161.29 90.17) (width 0.25) (layer F.Cu) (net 28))
 (segment (start 161.29 90.17) (end 160.02 88.9) (width 0.25) (layer F.Cu) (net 28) (status 800000))
 (segment (start 157.48 93.98) (end 157.48 93.472) (width 0.25) (layer F.Cu) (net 26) (status C00000))
 (segment (start 157.48 93.472) (end 158.75 92.202) (width 0.25) (layer F.Cu) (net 26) (status 400000))
 (segment (start 158.75 92.202) (end 158.75 90.17) (width 0.25) (layer F.Cu) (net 26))
 (segment (start 158.75 90.17) (end 157.48 88.9) (width 0.25) (layer F.Cu) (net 26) (status 800000))
 (segment (start 154.94 93.98) (end 154.94 93.472) (width 0.25) (layer F.Cu) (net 24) (status C00000))
 (segment (start 154.94 93.472) (end 156.21 92.202) (width 0.25) (layer F.Cu) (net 24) (status 400000))
 (segment (start 156.21 92.202) (end 156.21 90.17) (width 0.25) (layer F.Cu) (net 24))
 (segment (start 156.21 90.17) (end 154.94 88.9) (width 0.25) (layer F.Cu) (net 24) (status 800000))
 (segment (start 152.4 93.98) (end 152.4 93.472) (width 0.25) (layer F.Cu) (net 22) (status C00000))
 (segment (start 152.4 93.472) (end 153.67 92.202) (width 0.25) (layer F.Cu) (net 22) (status 400000))
 (segment (start 153.67 92.202) (end 153.67 90.17) (width 0.25) (layer F.Cu) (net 22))
 (segment (start 153.67 90.17) (end 152.4 88.9) (width 0.25) (layer F.Cu) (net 22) (status 800000))
 (segment (start 149.86 93.98) (end 149.86 93.472) (width 0.25) (layer F.Cu) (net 20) (status C00000))
 (segment (start 149.86 93.472) (end 151.13 92.202) (width 0.25) (layer F.Cu) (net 20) (status 400000))
 (segment (start 151.13 92.202) (end 151.13 90.17) (width 0.25) (layer F.Cu) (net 20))
 (segment (start 151.13 90.17) (end 149.86 88.9) (width 0.25) (layer F.Cu) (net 20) (status 800000))
 (segment (start 147.32 93.98) (end 147.32 93.472) (width 0.25) (layer F.Cu) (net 18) (status C00000))
 (segment (start 147.32 93.472) (end 148.59 92.202) (width 0.25) (layer F.Cu) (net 18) (status 400000))
 (segment (start 148.59 92.202) (end 148.59 90.17) (width 0.25) (layer F.Cu) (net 18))
 (segment (start 148.59 90.17) (end 147.32 88.9) (width 0.25) (layer F.Cu) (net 18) (status 800000))
 (segment (start 144.78 93.98) (end 144.78 93.472) (width 0.25) (layer F.Cu) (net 16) (status C00000))
 (segment (start 144.78 93.472) (end 146.05 92.202) (width 0.25) (layer F.Cu) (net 16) (status 400000))
 (segment (start 146.05 92.202) (end 146.05 90.17) (width 0.25) (layer F.Cu) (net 16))
 (segment (start 146.05 90.17) (end 144.78 88.9) (width 0.25) (layer F.Cu) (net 16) (status 800000))
 (segment (start 142.24 93.98) (end 142.24 93.472) (width 0.25) (layer F.Cu) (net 14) (status C00000))
 (segment (start 142.24 93.472) (end 143.51 92.202) (width 0.25) (layer F.Cu) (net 14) (status 400000))
 (segment (start 143.51 92.202) (end 143.51 90.17) (width 0.25) (layer F.Cu) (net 14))
 (segment (start 143.51 90.17) (end 142.24 88.9) (width 0.25) (layer F.Cu) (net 14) (status 800000))
 (segment (start 139.7 93.98) (end 139.7 93.597602) (width 0.25) (layer F.Cu) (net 12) (status C00000))
 (segment (start 139.7 93.597602) (end 140.97 92.327602) (width 0.25) (layer F.Cu) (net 12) (status 400000))
 (segment (start 140.97 92.327602) (end 140.97 90.17) (width 0.25) (layer F.Cu) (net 12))
 (segment (start 140.97 90.17) (end 139.7 88.9) (width 0.25) (layer F.Cu) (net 12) (status 800000))
 (segment (start 137.16 93.98) (end 137.16 93.472) (width 0.25) (layer F.Cu) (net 10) (status C00000))
 (segment (start 137.16 93.472) (end 138.43 92.202) (width 0.25) (layer F.Cu) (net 10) (status 400000))
 (segment (start 138.43 92.202) (end 138.43 90.17) (width 0.25) (layer F.Cu) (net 10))
 (segment (start 138.43 90.17) (end 137.16 88.9) (width 0.25) (layer F.Cu) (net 10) (status 800000))
 (segment (start 134.62 93.98) (end 134.62 93.472) (width 0.25) (layer F.Cu) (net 8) (status C00000))
 (segment (start 134.62 93.472) (end 135.89 92.202) (width 0.25) (layer F.Cu) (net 8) (status 400000))
 (segment (start 135.89 92.202) (end 135.89 90.17) (width 0.25) (layer F.Cu) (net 8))
 (segment (start 135.89 90.17) (end 134.62 88.9) (width 0.25) (layer F.Cu) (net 8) (status 800000))
 (segment (start 132.08 93.98) (end 132.08 93.472) (width 0.25) (layer F.Cu) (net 6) (status C00000))
 (segment (start 132.08 93.472) (end 133.35 92.202) (width 0.25) (layer F.Cu) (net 6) (status 400000))
 (segment (start 133.35 92.202) (end 133.35 90.17) (width 0.25) (layer F.Cu) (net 6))
 (segment (start 133.35 90.17) (end 132.08 88.9) (width 0.25) (layer F.Cu) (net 6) (status 800000))
 (segment (start 129.54 93.98) (end 129.54 93.472) (width 0.25) (layer F.Cu) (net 4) (status C00000))
 (segment (start 129.54 93.472) (end 130.81 92.202) (width 0.25) (layer F.Cu) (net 4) (status 400000))
 (segment (start 130.81 92.202) (end 130.81 90.17) (width 0.25) (layer F.Cu) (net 4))
 (segment (start 130.81 90.17) (end 129.54 88.9) (width 0.25) (layer F.Cu) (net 4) (status 800000))
 (segment (start 127 93.98) (end 127 93.726) (width 0.25) (layer F.Cu) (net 2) (status C00000))
 (segment (start 127 93.726) (end 128.27 92.456) (width 0.25) (layer F.Cu) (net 2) (status 400000))
 (segment (start 128.27 92.456) (end 128.27 90.17) (width 0.25) (layer F.Cu) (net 2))
 (segment (start 128.27 90.17) (end 127 88.9) (width 0.25) (layer F.Cu) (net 2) (status 800000)))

